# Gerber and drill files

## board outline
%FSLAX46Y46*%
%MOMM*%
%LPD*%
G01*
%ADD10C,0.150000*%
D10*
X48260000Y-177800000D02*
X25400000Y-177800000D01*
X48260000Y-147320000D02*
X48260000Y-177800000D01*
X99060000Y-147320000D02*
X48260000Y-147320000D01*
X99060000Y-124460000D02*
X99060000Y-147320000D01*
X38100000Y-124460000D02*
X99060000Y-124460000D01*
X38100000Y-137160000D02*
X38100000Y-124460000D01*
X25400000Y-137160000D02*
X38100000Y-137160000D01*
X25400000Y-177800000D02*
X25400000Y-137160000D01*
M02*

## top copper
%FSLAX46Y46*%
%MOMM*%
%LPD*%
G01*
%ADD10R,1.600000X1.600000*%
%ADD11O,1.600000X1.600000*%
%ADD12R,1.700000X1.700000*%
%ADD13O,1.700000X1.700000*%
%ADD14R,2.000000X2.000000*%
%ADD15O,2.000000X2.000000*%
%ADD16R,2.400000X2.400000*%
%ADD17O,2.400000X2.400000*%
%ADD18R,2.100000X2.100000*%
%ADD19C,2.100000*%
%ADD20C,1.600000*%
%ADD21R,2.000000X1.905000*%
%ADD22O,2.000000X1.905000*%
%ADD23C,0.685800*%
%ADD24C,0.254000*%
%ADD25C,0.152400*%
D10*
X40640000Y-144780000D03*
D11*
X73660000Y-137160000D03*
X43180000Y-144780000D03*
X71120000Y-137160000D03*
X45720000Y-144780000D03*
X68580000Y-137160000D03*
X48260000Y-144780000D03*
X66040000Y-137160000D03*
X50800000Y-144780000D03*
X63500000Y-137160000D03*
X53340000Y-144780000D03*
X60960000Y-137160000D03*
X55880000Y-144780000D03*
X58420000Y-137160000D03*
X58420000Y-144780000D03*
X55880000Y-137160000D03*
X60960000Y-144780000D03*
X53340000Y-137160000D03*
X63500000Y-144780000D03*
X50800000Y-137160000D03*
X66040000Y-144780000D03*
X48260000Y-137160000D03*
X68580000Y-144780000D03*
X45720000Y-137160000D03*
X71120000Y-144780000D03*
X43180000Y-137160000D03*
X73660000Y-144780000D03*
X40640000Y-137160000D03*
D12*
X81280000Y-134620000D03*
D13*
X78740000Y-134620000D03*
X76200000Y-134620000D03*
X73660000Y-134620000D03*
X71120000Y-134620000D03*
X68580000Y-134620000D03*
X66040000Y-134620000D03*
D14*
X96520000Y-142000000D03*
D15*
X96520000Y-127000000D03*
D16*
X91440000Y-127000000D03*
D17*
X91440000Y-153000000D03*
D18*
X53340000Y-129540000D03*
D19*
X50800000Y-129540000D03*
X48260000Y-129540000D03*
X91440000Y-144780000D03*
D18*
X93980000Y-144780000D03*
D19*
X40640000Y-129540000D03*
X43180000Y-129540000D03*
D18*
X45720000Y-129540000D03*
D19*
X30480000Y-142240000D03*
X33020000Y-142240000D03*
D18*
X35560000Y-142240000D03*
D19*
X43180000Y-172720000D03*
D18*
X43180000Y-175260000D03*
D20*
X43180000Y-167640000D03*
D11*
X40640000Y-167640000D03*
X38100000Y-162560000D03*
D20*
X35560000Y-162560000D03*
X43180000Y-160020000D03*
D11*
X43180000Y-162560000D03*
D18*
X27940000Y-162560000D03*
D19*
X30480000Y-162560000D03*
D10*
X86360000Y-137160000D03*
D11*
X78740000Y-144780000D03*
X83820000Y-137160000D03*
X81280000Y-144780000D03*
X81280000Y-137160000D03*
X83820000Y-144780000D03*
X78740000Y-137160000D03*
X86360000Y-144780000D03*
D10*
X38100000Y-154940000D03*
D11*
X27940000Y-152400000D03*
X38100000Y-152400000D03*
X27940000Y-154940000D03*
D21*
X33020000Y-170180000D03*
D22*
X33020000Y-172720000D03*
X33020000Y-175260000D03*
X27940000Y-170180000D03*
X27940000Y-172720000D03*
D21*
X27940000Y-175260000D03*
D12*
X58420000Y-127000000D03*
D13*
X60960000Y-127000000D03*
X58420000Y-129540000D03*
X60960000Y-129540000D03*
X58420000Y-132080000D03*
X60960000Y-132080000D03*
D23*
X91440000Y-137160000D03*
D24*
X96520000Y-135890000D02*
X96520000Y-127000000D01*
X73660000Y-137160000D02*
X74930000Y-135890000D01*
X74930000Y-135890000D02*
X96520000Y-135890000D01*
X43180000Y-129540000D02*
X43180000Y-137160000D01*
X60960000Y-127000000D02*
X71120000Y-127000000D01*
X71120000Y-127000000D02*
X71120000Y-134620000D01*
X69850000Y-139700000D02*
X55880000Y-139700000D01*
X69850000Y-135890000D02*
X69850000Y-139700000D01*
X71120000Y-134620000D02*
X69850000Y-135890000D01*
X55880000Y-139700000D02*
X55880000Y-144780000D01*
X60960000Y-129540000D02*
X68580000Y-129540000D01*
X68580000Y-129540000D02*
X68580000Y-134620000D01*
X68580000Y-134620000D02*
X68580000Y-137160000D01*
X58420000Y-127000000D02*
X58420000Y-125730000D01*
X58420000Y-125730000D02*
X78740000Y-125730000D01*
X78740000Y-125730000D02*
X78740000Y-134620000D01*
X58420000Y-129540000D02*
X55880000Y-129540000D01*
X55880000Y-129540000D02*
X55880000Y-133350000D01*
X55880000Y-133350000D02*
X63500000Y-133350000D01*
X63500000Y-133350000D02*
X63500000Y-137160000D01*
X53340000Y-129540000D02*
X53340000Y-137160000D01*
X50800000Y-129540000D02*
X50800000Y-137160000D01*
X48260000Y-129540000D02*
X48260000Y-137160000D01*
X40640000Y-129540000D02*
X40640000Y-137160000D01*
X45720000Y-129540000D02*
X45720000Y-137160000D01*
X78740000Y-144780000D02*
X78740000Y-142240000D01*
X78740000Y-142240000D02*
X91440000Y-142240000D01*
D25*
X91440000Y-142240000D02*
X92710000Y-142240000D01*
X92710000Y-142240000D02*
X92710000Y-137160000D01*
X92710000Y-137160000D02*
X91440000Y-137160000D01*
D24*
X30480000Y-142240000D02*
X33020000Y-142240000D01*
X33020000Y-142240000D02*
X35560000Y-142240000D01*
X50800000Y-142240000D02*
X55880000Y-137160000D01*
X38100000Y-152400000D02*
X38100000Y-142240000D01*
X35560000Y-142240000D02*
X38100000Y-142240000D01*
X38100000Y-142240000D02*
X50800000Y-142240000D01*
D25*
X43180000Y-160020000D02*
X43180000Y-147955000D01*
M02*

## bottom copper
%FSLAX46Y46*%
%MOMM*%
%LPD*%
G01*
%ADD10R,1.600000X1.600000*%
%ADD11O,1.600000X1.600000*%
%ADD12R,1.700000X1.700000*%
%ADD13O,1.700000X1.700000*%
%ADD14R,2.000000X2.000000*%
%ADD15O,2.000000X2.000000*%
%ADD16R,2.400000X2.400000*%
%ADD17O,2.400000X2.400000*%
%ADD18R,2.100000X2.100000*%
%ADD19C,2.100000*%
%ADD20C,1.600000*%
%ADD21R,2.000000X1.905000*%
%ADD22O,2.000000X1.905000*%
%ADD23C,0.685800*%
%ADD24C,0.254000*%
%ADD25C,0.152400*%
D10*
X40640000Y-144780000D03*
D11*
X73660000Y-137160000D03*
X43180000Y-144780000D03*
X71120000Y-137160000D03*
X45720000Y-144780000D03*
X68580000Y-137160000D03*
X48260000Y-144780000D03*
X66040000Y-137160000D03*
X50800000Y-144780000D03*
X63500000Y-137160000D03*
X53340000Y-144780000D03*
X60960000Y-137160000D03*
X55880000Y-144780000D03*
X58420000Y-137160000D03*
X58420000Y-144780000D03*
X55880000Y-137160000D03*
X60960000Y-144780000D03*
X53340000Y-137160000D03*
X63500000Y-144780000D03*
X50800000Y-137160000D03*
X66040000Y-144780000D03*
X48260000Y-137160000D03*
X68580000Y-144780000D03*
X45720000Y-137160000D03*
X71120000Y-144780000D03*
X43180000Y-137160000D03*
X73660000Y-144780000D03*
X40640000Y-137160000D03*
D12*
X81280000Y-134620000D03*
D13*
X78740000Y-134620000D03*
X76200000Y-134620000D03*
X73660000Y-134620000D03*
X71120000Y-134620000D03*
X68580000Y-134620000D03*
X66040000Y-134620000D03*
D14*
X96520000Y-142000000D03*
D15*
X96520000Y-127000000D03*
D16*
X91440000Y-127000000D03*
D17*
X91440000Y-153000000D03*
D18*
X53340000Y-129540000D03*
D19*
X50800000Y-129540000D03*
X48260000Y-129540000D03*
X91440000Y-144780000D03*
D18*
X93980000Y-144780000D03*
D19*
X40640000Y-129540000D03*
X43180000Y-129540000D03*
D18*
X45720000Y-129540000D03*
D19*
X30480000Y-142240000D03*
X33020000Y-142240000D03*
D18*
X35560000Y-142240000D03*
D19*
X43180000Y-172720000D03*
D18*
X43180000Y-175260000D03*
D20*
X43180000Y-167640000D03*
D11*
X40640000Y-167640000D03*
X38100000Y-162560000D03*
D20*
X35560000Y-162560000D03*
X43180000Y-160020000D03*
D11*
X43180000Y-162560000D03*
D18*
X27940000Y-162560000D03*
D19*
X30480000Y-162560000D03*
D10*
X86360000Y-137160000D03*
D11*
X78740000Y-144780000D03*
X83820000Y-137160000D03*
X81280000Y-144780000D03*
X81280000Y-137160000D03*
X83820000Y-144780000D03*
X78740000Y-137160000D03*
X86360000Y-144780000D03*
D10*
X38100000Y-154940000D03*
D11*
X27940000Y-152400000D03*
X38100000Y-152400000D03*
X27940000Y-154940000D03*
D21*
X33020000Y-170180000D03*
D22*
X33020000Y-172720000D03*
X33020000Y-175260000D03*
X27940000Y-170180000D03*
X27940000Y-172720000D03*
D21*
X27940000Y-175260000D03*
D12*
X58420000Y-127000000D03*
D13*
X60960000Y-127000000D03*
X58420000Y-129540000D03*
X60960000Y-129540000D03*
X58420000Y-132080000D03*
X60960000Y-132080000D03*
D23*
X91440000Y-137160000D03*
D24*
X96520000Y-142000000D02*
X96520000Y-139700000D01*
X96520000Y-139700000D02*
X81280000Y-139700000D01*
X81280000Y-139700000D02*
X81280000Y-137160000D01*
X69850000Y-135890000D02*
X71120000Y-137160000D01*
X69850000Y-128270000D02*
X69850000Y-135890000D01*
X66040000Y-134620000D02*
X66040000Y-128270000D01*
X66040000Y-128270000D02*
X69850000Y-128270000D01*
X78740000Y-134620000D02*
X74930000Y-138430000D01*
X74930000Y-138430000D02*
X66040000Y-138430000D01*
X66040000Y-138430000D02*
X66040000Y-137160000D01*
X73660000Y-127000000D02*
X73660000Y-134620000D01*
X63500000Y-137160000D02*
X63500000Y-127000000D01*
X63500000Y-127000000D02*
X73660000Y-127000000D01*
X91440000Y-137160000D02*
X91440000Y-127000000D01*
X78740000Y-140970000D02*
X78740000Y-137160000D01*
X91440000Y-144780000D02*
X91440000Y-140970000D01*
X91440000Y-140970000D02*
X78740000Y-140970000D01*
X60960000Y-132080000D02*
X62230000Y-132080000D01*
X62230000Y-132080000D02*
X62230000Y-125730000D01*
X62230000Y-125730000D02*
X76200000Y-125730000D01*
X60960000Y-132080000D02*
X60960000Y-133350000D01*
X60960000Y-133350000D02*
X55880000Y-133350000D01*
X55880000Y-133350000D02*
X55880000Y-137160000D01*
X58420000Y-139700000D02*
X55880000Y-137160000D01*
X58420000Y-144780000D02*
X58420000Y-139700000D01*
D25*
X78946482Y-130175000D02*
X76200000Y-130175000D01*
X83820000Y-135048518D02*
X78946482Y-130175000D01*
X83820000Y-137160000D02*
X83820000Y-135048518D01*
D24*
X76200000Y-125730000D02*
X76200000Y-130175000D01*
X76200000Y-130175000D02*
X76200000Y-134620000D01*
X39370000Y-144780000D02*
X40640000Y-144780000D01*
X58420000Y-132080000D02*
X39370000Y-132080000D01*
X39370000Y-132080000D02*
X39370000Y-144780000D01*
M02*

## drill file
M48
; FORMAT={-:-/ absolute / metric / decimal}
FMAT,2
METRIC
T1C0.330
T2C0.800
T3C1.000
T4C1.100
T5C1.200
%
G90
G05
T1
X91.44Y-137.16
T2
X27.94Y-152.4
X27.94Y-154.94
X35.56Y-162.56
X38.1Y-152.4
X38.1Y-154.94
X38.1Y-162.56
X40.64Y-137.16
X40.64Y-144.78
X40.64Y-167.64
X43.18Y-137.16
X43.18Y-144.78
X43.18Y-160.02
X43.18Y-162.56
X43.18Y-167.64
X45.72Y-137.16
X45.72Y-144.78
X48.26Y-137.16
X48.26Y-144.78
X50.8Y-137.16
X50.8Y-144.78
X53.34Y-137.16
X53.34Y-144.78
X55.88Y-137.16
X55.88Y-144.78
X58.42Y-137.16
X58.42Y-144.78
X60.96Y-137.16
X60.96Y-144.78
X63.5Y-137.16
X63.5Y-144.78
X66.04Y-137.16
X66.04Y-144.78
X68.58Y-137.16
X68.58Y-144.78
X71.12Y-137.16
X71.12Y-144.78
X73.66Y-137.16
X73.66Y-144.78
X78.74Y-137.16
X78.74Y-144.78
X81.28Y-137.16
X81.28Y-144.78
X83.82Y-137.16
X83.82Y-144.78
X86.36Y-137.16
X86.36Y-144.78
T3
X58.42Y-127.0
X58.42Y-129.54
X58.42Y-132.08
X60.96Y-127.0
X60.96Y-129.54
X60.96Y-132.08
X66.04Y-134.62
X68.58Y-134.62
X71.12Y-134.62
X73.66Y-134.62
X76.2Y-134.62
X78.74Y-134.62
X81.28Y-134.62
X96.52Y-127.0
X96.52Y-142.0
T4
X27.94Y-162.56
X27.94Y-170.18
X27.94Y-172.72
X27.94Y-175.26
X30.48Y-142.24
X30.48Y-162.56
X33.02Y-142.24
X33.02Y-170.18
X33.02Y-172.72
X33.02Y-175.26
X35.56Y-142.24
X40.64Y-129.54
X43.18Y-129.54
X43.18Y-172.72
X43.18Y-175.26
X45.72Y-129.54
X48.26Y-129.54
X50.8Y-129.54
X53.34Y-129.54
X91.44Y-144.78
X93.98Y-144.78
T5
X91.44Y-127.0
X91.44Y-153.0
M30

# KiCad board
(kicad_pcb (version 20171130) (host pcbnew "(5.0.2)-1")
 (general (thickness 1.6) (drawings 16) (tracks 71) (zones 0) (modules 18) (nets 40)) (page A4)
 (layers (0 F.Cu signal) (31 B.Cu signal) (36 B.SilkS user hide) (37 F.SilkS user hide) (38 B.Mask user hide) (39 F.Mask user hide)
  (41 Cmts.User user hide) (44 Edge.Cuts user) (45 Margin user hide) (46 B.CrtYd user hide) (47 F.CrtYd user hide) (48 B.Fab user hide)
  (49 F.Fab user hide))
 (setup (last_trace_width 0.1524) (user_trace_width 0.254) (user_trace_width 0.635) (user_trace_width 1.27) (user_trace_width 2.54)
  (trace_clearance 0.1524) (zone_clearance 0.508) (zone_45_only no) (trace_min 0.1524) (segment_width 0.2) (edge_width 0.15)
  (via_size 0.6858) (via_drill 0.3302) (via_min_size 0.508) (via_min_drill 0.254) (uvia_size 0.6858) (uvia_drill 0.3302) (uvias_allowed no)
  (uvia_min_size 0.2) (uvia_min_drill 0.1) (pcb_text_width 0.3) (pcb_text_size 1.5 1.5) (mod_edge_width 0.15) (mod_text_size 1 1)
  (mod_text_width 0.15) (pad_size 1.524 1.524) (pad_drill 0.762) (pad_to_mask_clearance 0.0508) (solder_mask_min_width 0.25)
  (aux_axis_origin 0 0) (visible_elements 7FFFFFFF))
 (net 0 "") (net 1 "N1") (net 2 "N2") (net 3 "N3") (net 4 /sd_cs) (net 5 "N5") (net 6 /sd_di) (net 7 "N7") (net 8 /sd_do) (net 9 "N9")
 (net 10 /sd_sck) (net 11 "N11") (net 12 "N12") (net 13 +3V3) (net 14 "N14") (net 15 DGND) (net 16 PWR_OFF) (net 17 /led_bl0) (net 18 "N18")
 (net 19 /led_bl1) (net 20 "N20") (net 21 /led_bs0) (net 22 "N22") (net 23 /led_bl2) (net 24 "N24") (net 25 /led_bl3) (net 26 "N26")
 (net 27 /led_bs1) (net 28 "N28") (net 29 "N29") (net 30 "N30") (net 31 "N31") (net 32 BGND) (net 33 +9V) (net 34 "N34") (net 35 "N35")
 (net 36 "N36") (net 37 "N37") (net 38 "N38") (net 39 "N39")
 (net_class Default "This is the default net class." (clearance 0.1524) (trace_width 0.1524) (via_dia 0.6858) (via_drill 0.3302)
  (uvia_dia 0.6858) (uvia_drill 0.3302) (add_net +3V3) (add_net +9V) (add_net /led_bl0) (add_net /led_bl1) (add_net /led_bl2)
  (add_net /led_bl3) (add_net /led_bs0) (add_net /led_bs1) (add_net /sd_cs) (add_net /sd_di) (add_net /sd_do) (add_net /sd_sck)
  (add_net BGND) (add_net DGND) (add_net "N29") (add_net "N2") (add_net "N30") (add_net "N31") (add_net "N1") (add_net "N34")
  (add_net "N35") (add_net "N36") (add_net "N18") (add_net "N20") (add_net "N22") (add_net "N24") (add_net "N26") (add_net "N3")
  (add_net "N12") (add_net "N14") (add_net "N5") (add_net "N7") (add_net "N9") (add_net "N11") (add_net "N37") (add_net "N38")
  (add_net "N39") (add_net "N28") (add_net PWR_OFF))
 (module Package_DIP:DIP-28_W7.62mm (layer F.Cu) (at 40.64 144.78 90)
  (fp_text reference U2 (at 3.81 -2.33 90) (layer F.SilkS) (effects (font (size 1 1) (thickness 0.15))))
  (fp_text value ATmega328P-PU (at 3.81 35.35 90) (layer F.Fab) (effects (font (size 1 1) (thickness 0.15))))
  (pad 1 thru_hole rect (at 0 0 90) (size 1.6 1.6) (drill 0.8) (layers *.Cu *.Mask) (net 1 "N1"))
  (pad 15 thru_hole oval (at 7.62 33.02 90) (size 1.6 1.6) (drill 0.8) (layers *.Cu *.Mask) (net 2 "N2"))
  (pad 2 thru_hole oval (at 0 2.54 90) (size 1.6 1.6) (drill 0.8) (layers *.Cu *.Mask) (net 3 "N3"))
  (pad 16 thru_hole oval (at 7.62 30.48 90) (size 1.6 1.6) (drill 0.8) (layers *.Cu *.Mask) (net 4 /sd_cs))
  (pad 3 thru_hole oval (at 0 5.08 90) (size 1.6 1.6) (drill 0.8) (layers *.Cu *.Mask) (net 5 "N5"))
  (pad 17 thru_hole oval (at 7.62 27.94 90) (size 1.6 1.6) (drill 0.8) (layers *.Cu *.Mask) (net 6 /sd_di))
  (pad 4 thru_hole oval (at 0 7.62 90) (size 1.6 1.6) (drill 0.8) (layers *.Cu *.Mask) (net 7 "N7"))
  (pad 18 thru_hole oval (at 7.62 25.4 90) (size 1.6 1.6) (drill 0.8) (layers *.Cu *.Mask) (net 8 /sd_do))
  (pad 5 thru_hole oval (at 0 10.16 90) (size 1.6 1.6) (drill 0.8) (layers *.Cu *.Mask) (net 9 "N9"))
  (pad 19 thru_hole oval (at 7.62 22.86 90) (size 1.6 1.6) (drill 0.8) (layers *.Cu *.Mask) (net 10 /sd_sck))
  (pad 6 thru_hole oval (at 0 12.7 90) (size 1.6 1.6) (drill 0.8) (layers *.Cu *.Mask) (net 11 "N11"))
  (pad 20 thru_hole oval (at 7.62 20.32 90) (size 1.6 1.6) (drill 0.8) (layers *.Cu *.Mask) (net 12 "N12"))
  (pad 7 thru_hole oval (at 0 15.24 90) (size 1.6 1.6) (drill 0.8) (layers *.Cu *.Mask) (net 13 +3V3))
  (pad 21 thru_hole oval (at 7.62 17.78 90) (size 1.6 1.6) (drill 0.8) (layers *.Cu *.Mask) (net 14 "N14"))
  (pad 8 thru_hole oval (at 0 17.78 90) (size 1.6 1.6) (drill 0.8) (layers *.Cu *.Mask) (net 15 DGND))
  (pad 22 thru_hole oval (at 7.62 15.24 90) (size 1.6 1.6) (drill 0.8) (layers *.Cu *.Mask) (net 15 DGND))
  (pad 9 thru_hole oval (at 0 20.32 90) (size 1.6 1.6) (drill 0.8) (layers *.Cu *.Mask) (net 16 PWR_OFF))
  (pad 23 thru_hole oval (at 7.62 12.7 90) (size 1.6 1.6) (drill 0.8) (layers *.Cu *.Mask) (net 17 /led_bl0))
  (pad 10 thru_hole oval (at 0 22.86 90) (size 1.6 1.6) (drill 0.8) (layers *.Cu *.Mask) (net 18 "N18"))
  (pad 24 thru_hole oval (at 7.62 10.16 90) (size 1.6 1.6) (drill 0.8) (layers *.Cu *.Mask) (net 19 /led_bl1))
  (pad 11 thru_hole oval (at 0 25.4 90) (size 1.6 1.6) (drill 0.8) (layers *.Cu *.Mask) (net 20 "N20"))
  (pad 25 thru_hole oval (at 7.62 7.62 90) (size 1.6 1.6) (drill 0.8) (layers *.Cu *.Mask) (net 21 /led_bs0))
  (pad 12 thru_hole oval (at 0 27.94 90) (size 1.6 1.6) (drill 0.8) (layers *.Cu *.Mask) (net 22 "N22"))
  (pad 26 thru_hole oval (at 7.62 5.08 90) (size 1.6 1.6) (drill 0.8) (layers *.Cu *.Mask) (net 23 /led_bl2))
  (pad 13 thru_hole oval (at 0 30.48 90) (size 1.6 1.6) (drill 0.8) (layers *.Cu *.Mask) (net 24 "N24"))
  (pad 27 thru_hole oval (at 7.62 2.54 90) (size 1.6 1.6) (drill 0.8) (layers *.Cu *.Mask) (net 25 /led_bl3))
  (pad 14 thru_hole oval (at 0 33.02 90) (size 1.6 1.6) (drill 0.8) (layers *.Cu *.Mask) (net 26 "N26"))
  (pad 28 thru_hole oval (at 7.62 0 90) (size 1.6 1.6) (drill 0.8) (layers *.Cu *.Mask) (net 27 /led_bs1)))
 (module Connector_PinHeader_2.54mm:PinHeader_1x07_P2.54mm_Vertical (layer F.Cu) (at 81.28 134.62 270)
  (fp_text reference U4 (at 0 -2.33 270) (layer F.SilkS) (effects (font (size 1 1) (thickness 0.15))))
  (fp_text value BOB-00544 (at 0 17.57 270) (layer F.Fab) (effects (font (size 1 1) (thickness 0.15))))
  (pad 1 thru_hole rect (at 0 0 270) (size 1.7 1.7) (drill 1) (layers *.Cu *.Mask) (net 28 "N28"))
  (pad 2 thru_hole oval (at 0 2.54 270) (size 1.7 1.7) (drill 1) (layers *.Cu *.Mask) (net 8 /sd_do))
  (pad 3 thru_hole oval (at 0 5.08 270) (size 1.7 1.7) (drill 1) (layers *.Cu *.Mask) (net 15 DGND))
  (pad 4 thru_hole oval (at 0 7.62 270) (size 1.7 1.7) (drill 1) (layers *.Cu *.Mask) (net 10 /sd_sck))
  (pad 5 thru_hole oval (at 0 10.16 270) (size 1.7 1.7) (drill 1) (layers *.Cu *.Mask) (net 13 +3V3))
  (pad 6 thru_hole oval (at 0 12.7 270) (size 1.7 1.7) (drill 1) (layers *.Cu *.Mask) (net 6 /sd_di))
  (pad 7 thru_hole oval (at 0 15.24 270) (size 1.7 1.7) (drill 1) (layers *.Cu *.Mask) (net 4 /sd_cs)))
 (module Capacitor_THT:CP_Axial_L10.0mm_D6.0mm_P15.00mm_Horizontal (layer F.Cu) (at 96.52 142 90)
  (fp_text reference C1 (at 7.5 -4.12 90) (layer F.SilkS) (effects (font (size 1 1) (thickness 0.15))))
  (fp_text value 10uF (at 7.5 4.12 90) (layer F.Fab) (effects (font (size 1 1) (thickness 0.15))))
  (pad 1 thru_hole rect (at 0 0 90) (size 2 2) (drill 1) (layers *.Cu *.Mask) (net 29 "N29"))
  (pad 2 thru_hole oval (at 15 0 90) (size 2 2) (drill 1) (layers *.Cu *.Mask) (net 2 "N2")))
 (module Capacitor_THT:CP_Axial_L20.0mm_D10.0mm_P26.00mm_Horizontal (layer F.Cu) (at 91.44 127 270)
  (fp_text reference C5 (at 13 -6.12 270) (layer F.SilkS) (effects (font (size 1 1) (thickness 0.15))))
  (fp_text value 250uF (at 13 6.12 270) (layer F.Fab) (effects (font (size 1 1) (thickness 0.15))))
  (pad 1 thru_hole rect (at 0 0 270) (size 2.4 2.4) (drill 1.2) (layers *.Cu *.Mask) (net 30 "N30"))
  (pad 2 thru_hole oval (at 26 0 270) (size 2.4 2.4) (drill 1.2) (layers *.Cu *.Mask) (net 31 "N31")))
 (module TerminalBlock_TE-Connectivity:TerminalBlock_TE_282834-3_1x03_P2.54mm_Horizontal (layer F.Cu) (at 53.34 129.54 180)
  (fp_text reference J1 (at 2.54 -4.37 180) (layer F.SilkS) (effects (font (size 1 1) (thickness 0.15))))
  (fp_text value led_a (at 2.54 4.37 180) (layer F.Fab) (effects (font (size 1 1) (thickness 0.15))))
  (pad 1 thru_hole rect (at 0 0 180) (size 2.1 2.1) (drill 1.1) (layers *.Cu *.Mask) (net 17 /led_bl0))
  (pad 2 thru_hole circle (at 2.54 0 180) (size 2.1 2.1) (drill 1.1) (layers *.Cu *.Mask) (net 19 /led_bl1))
  (pad 3 thru_hole circle (at 5.08 0 180) (size 2.1 2.1) (drill 1.1) (layers *.Cu *.Mask) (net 21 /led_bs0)))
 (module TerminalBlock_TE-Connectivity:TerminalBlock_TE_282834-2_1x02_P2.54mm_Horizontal (layer F.Cu) (at 93.98 144.78 180)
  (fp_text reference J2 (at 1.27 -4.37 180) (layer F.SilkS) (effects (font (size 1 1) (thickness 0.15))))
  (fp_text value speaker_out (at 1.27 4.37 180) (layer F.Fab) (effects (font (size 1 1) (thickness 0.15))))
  (pad 2 thru_hole circle (at 2.54 0 180) (size 2.1 2.1) (drill 1.1) (layers *.Cu *.Mask) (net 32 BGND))
  (pad 1 thru_hole rect (at 0 0 180) (size 2.1 2.1) (drill 1.1) (layers *.Cu *.Mask) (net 31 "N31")))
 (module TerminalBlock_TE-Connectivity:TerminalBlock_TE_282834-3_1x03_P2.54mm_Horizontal (layer F.Cu) (at 45.72 129.54 180)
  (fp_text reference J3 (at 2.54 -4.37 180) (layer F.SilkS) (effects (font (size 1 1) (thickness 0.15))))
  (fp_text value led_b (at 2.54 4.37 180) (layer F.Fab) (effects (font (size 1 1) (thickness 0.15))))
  (pad 3 thru_hole circle (at 5.08 0 180) (size 2.1 2.1) (drill 1.1) (layers *.Cu *.Mask) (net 27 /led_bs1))
  (pad 2 thru_hole circle (at 2.54 0 180) (size 2.1 2.1) (drill 1.1) (layers *.Cu *.Mask) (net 25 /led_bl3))
  (pad 1 thru_hole rect (at 0 0 180) (size 2.1 2.1) (drill 1.1) (layers *.Cu *.Mask) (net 23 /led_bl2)))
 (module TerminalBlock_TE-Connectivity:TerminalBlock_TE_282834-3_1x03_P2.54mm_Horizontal (layer F.Cu) (at 35.56 142.24 180)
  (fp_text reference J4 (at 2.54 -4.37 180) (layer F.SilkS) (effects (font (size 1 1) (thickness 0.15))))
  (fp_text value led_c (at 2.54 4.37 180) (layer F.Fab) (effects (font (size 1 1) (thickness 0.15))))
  (pad 3 thru_hole circle (at 5.08 0 180) (size 2.1 2.1) (drill 1.1) (layers *.Cu *.Mask) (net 15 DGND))
  (pad 2 thru_hole circle (at 2.54 0 180) (size 2.1 2.1) (drill 1.1) (layers *.Cu *.Mask) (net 15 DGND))
  (pad 1 thru_hole rect (at 0 0 180) (size 2.1 2.1) (drill 1.1) (layers *.Cu *.Mask) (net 15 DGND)))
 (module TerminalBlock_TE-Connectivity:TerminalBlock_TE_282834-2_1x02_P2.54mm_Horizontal (layer F.Cu) (at 43.18 175.26 90)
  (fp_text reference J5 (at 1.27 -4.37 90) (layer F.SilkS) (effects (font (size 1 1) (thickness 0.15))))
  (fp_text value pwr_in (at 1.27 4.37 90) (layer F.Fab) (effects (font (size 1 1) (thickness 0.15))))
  (pad 2 thru_hole circle (at 2.54 0 90) (size 2.1 2.1) (drill 1.1) (layers *.Cu *.Mask) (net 32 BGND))
  (pad 1 thru_hole rect (at 0 0 90) (size 2.1 2.1) (drill 1.1) (layers *.Cu *.Mask) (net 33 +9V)))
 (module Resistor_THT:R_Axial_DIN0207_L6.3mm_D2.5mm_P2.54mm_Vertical (layer F.Cu) (at 43.18 167.64 180)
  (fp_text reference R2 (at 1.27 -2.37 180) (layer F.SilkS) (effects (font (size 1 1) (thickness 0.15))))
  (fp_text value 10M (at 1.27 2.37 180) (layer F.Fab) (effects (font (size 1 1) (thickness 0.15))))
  (pad 1 thru_hole circle (at 0 0 180) (size 1.6 1.6) (drill 0.8) (layers *.Cu *.Mask) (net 33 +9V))
  (pad 2 thru_hole oval (at 2.54 0 180) (size 1.6 1.6) (drill 0.8) (layers *.Cu *.Mask) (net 15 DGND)))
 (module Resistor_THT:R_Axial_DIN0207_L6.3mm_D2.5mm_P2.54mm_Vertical (layer F.Cu) (at 35.56 162.56)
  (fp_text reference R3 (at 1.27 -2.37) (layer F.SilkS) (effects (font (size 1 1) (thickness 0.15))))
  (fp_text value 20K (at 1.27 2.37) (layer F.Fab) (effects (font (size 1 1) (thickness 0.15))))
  (pad 2 thru_hole oval (at 2.54 0) (size 1.6 1.6) (drill 0.8) (layers *.Cu *.Mask) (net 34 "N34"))
  (pad 1 thru_hole circle (at 0 0) (size 1.6 1.6) (drill 0.8) (layers *.Cu *.Mask) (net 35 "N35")))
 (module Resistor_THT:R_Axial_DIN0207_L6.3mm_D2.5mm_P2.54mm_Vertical (layer F.Cu) (at 43.18 160.02 270)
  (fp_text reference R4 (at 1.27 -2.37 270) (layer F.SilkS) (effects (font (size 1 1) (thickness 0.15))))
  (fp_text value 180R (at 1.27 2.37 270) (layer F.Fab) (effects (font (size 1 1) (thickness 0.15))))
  (pad 1 thru_hole circle (at 0 0 270) (size 1.6 1.6) (drill 0.8) (layers *.Cu *.Mask) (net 16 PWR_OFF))
  (pad 2 thru_hole oval (at 2.54 0 270) (size 1.6 1.6) (drill 0.8) (layers *.Cu *.Mask) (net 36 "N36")))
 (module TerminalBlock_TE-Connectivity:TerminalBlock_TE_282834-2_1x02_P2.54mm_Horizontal (layer F.Cu) (at 27.94 162.56)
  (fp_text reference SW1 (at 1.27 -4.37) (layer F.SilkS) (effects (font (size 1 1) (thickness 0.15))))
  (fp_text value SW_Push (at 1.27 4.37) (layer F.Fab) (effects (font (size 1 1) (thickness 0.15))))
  (pad 1 thru_hole rect (at 0 0) (size 2.1 2.1) (drill 1.1) (layers *.Cu *.Mask) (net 33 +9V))
  (pad 2 thru_hole circle (at 2.54 0) (size 2.1 2.1) (drill 1.1) (layers *.Cu *.Mask) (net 35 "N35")))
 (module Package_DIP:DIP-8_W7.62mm (layer F.Cu) (at 86.36 137.16 270)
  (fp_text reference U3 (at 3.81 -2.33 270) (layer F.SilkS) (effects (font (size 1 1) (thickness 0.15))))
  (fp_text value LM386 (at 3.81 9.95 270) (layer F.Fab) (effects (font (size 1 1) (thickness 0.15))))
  (pad 1 thru_hole rect (at 0 0 270) (size 1.6 1.6) (drill 0.8) (layers *.Cu *.Mask) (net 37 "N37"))
  (pad 5 thru_hole oval (at 7.62 7.62 270) (size 1.6 1.6) (drill 0.8) (layers *.Cu *.Mask) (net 30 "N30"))
  (pad 2 thru_hole oval (at 0 2.54 270) (size 1.6 1.6) (drill 0.8) (layers *.Cu *.Mask) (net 15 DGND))
  (pad 6 thru_hole oval (at 7.62 5.08 270) (size 1.6 1.6) (drill 0.8) (layers *.Cu *.Mask) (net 33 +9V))
  (pad 3 thru_hole oval (at 0 5.08 270) (size 1.6 1.6) (drill 0.8) (layers *.Cu *.Mask) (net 29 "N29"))
  (pad 7 thru_hole oval (at 7.62 2.54 270) (size 1.6 1.6) (drill 0.8) (layers *.Cu *.Mask) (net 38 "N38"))
  (pad 4 thru_hole oval (at 0 7.62 270) (size 1.6 1.6) (drill 0.8) (layers *.Cu *.Mask) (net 32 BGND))
  (pad 8 thru_hole oval (at 7.62 0 270) (size 1.6 1.6) (drill 0.8) (layers *.Cu *.Mask) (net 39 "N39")))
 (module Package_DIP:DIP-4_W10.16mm (layer F.Cu) (at 38.1 154.94 180)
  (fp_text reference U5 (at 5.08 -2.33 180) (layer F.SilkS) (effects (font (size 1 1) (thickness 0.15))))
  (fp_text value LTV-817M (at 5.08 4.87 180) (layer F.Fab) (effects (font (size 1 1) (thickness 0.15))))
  (pad 1 thru_hole rect (at 0 0 180) (size 1.6 1.6) (drill 0.8) (layers *.Cu *.Mask) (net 36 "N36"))
  (pad 3 thru_hole oval (at 10.16 2.54 180) (size 1.6 1.6) (drill 0.8) (layers *.Cu *.Mask) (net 32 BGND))
  (pad 2 thru_hole oval (at 0 2.54 180) (size 1.6 1.6) (drill 0.8) (layers *.Cu *.Mask) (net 15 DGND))
  (pad 4 thru_hole oval (at 10.16 0 180) (size 1.6 1.6) (drill 0.8) (layers *.Cu *.Mask) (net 34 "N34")))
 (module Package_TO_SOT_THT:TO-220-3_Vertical (layer F.Cu) (at 33.02 170.18 270)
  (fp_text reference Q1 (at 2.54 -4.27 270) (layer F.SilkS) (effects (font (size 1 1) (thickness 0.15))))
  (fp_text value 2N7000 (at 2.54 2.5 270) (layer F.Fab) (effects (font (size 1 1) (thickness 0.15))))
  (pad 1 thru_hole rect (at 0 0 270) (size 1.905 2) (drill 1.1) (layers *.Cu *.Mask) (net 32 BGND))
  (pad 2 thru_hole oval (at 2.54 0 270) (size 1.905 2) (drill 1.1) (layers *.Cu *.Mask) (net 34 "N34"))
  (pad 3 thru_hole oval (at 5.08 0 270) (size 1.905 2) (drill 1.1) (layers *.Cu *.Mask) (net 15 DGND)))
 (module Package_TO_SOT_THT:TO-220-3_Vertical (layer F.Cu) (at 27.94 175.26 90)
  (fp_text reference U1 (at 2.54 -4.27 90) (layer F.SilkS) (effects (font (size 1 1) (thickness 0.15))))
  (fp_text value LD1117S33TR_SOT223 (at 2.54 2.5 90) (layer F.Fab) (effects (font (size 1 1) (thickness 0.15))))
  (pad 3 thru_hole oval (at 5.08 0 90) (size 1.905 2) (drill 1.1) (layers *.Cu *.Mask) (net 33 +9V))
  (pad 2 thru_hole oval (at 2.54 0 90) (size 1.905 2) (drill 1.1) (layers *.Cu *.Mask) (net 13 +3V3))
  (pad 1 thru_hole rect (at 0 0 90) (size 1.905 2) (drill 1.1) (layers *.Cu *.Mask) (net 15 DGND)))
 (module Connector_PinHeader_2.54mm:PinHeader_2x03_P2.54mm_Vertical (layer F.Cu) (at 58.42 127)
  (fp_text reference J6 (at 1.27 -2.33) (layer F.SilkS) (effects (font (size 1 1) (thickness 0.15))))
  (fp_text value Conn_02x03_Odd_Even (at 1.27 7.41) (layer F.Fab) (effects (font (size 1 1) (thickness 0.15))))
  (pad 1 thru_hole rect (at 0 0) (size 1.7 1.7) (drill 1) (layers *.Cu *.Mask) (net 8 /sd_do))
  (pad 2 thru_hole oval (at 2.54 0) (size 1.7 1.7) (drill 1) (layers *.Cu *.Mask) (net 13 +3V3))
  (pad 3 thru_hole oval (at 0 2.54) (size 1.7 1.7) (drill 1) (layers *.Cu *.Mask) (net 10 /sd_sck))
  (pad 4 thru_hole oval (at 2.54 2.54) (size 1.7 1.7) (drill 1) (layers *.Cu *.Mask) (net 6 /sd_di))
  (pad 5 thru_hole oval (at 0 5.08) (size 1.7 1.7) (drill 1) (layers *.Cu *.Mask) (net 1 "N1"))
  (pad 6 thru_hole oval (at 2.54 5.08) (size 1.7 1.7) (drill 1) (layers *.Cu *.Mask) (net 15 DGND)))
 (gr_line (start 48.26 177.8) (end 25.4 177.8) (layer Edge.Cuts) (width 0.15))
 (gr_line (start 48.26 147.32) (end 48.26 177.8) (layer Edge.Cuts) (width 0.15))
 (gr_line (start 99.06 147.32) (end 48.26 147.32) (layer Edge.Cuts) (width 0.15))
 (gr_line (start 99.06 124.46) (end 99.06 147.32) (layer Edge.Cuts) (width 0.15))
 (gr_line (start 38.1 124.46) (end 99.06 124.46) (layer Edge.Cuts) (width 0.15))
 (gr_line (start 38.1 137.16) (end 38.1 124.46) (layer Edge.Cuts) (width 0.15))
 (gr_line (start 25.4 137.16) (end 38.1 137.16) (layer Edge.Cuts) (width 0.15))
 (gr_line (start 25.4 177.8) (end 25.4 137.16) (layer Edge.Cuts) (width 0.15))
 (segment (start 96.52 142) (end 96.52 139.7) (width 0.254) (layer B.Cu) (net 29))
 (segment (start 96.52 139.7) (end 81.28 139.7) (width 0.254) (layer B.Cu) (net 29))
 (segment (start 81.28 139.7) (end 81.28 137.16) (width 0.254) (layer B.Cu) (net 29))
 (segment (start 96.52 135.89) (end 96.52 127) (width 0.254) (layer F.Cu) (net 2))
 (segment (start 73.66 137.16) (end 74.93 135.89) (width 0.254) (layer F.Cu) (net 2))
 (segment (start 74.93 135.89) (end 96.52 135.89) (width 0.254) (layer F.Cu) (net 2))
 (segment (start 43.18 129.54) (end 43.18 137.16) (width 0.254) (layer F.Cu) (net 25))
 (segment (start 60.96 127) (end 71.12 127) (width 0.254) (layer F.Cu) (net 13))
 (segment (start 71.12 127) (end 71.12 134.62) (width 0.254) (layer F.Cu) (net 13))
 (segment (start 69.85 139.7) (end 55.88 139.7) (width 0.254) (layer F.Cu) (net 13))
 (segment (start 69.85 135.89) (end 69.85 139.7) (width 0.254) (layer F.Cu) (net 13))
 (segment (start 71.12 134.62) (end 69.85 135.89) (width 0.254) (layer F.Cu) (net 13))
 (segment (start 55.88 139.7) (end 55.88 144.78) (width 0.254) (layer F.Cu) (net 13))
 (segment (start 69.85 135.89) (end 71.12 137.16) (width 0.254) (layer B.Cu) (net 4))
 (segment (start 69.85 128.27) (end 69.85 135.89) (width 0.254) (layer B.Cu) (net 4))
 (segment (start 66.04 134.62) (end 66.04 128.27) (width 0.254) (layer B.Cu) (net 4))
 (segment (start 66.04 128.27) (end 69.85 128.27) (width 0.254) (layer B.Cu) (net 4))
 (segment (start 60.96 129.54) (end 68.58 129.54) (width 0.254) (layer F.Cu) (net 6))
 (segment (start 68.58 129.54) (end 68.58 134.62) (width 0.254) (layer F.Cu) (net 6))
 (segment (start 68.58 134.62) (end 68.58 137.16) (width 0.254) (layer F.Cu) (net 6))
 (segment (start 58.42 127) (end 58.42 125.73) (width 0.254) (layer F.Cu) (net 8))
 (segment (start 58.42 125.73) (end 78.74 125.73) (width 0.254) (layer F.Cu) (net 8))
 (segment (start 78.74 125.73) (end 78.74 134.62) (width 0.254) (layer F.Cu) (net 8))
 (segment (start 78.74 134.62) (end 74.93 138.43) (width 0.254) (layer B.Cu) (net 8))
 (segment (start 74.93 138.43) (end 66.04 138.43) (width 0.254) (layer B.Cu) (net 8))
 (segment (start 66.04 138.43) (end 66.04 137.16) (width 0.254) (layer B.Cu) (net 8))
 (segment (start 73.66 127) (end 73.66 134.62) (width 0.254) (layer B.Cu) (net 10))
 (segment (start 63.5 137.16) (end 63.5 127) (width 0.254) (layer B.Cu) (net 10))
 (segment (start 63.5 127) (end 73.66 127) (width 0.254) (layer B.Cu) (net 10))
 (segment (start 58.42 129.54) (end 55.88 129.54) (width 0.254) (layer F.Cu) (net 10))
 (segment (start 55.88 129.54) (end 55.88 133.35) (width 0.254) (layer F.Cu) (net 10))
 (segment (start 55.88 133.35) (end 63.5 133.35) (width 0.254) (layer F.Cu) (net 10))
 (segment (start 63.5 133.35) (end 63.5 137.16) (width 0.254) (layer F.Cu) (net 10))
 (segment (start 53.34 129.54) (end 53.34 137.16) (width 0.254) (layer F.Cu) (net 17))
 (segment (start 50.8 129.54) (end 50.8 137.16) (width 0.254) (layer F.Cu) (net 19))
 (segment (start 48.26 129.54) (end 48.26 137.16) (width 0.254) (layer F.Cu) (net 21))
 (segment (start 40.64 129.54) (end 40.64 137.16) (width 0.254) (layer F.Cu) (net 27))
 (segment (start 45.72 129.54) (end 45.72 137.16) (width 0.254) (layer F.Cu) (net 23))
 (segment (start 78.74 144.78) (end 78.74 142.24) (width 0.254) (layer F.Cu) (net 30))
 (segment (start 78.74 142.24) (end 91.44 142.24) (width 0.254) (layer F.Cu) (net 30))
 (via (at 91.44 137.16) (size 0.6858) (drill 0.3302) (layers F.Cu B.Cu) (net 30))
 (segment (start 91.44 137.16) (end 91.44 127) (width 0.254) (layer B.Cu) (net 30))
 (segment (start 91.44 142.24) (end 92.71 142.24) (width 0.1524) (layer F.Cu) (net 30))
 (segment (start 92.71 142.24) (end 92.71 137.16) (width 0.1524) (layer F.Cu) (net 30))
 (segment (start 92.71 137.16) (end 91.44 137.16) (width 0.1524) (layer F.Cu) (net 30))
 (segment (start 78.74 140.97) (end 78.74 137.16) (width 0.254) (layer B.Cu) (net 32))
 (segment (start 91.44 144.78) (end 91.44 140.97) (width 0.254) (layer B.Cu) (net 32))
 (segment (start 91.44 140.97) (end 78.74 140.97) (width 0.254) (layer B.Cu) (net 32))
 (segment (start 60.96 132.08) (end 62.23 132.08) (width 0.254) (layer B.Cu) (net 15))
 (segment (start 62.23 132.08) (end 62.23 125.73) (width 0.254) (layer B.Cu) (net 15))
 (segment (start 62.23 125.73) (end 76.2 125.73) (width 0.254) (layer B.Cu) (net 15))
 (segment (start 60.96 132.08) (end 60.96 133.35) (width 0.254) (layer B.Cu) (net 15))
 (segment (start 60.96 133.35) (end 55.88 133.35) (width 0.254) (layer B.Cu) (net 15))
 (segment (start 55.88 133.35) (end 55.88 137.16) (width 0.254) (layer B.Cu) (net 15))
 (segment (start 58.42 139.7) (end 55.88 137.16) (width 0.254) (layer B.Cu) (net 15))
 (segment (start 58.42 144.78) (end 58.42 139.7) (width 0.254) (layer B.Cu) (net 15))
 (segment (start 30.48 142.24) (end 33.02 142.24) (width 0.254) (layer F.Cu) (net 15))
 (segment (start 33.02 142.24) (end 35.56 142.24) (width 0.254) (layer F.Cu) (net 15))
 (segment (start 50.8 142.24) (end 55.88 137.16) (width 0.254) (layer F.Cu) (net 15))
 (segment (start 38.1 152.4) (end 38.1 142.24) (width 0.254) (layer F.Cu) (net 15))
 (segment (start 35.56 142.24) (end 38.1 142.24) (width 0.254) (layer F.Cu) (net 15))
 (segment (start 38.1 142.24) (end 50.8 142.24) (width 0.254) (layer F.Cu) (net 15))
 (segment (start 78.946482 130.175) (end 76.2 130.175) (width 0.1524) (layer B.Cu) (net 15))
 (segment (start 83.82 135.048518) (end 78.946482 130.175) (width 0.1524) (layer B.Cu) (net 15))
 (segment (start 83.82 137.16) (end 83.82 135.048518) (width 0.1524) (layer B.Cu) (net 15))
 (segment (start 76.2 125.73) (end 76.2 130.175) (width 0.254) (layer B.Cu) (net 15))
 (segment (start 76.2 130.175) (end 76.2 134.62) (width 0.254) (layer B.Cu) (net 15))
 (segment (start 43.18 160.02) (end 43.18 147.955) (width 0.1524) (layer F.Cu) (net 16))
 (segment (start 39.37 144.78) (end 40.64 144.78) (width 0.254) (layer B.Cu) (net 1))
 (segment (start 58.42 132.08) (end 39.37 132.08) (width 0.254) (layer B.Cu) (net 1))
 (segment (start 39.37 132.08) (end 39.37 144.78) (width 0.254) (layer B.Cu) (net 1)))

